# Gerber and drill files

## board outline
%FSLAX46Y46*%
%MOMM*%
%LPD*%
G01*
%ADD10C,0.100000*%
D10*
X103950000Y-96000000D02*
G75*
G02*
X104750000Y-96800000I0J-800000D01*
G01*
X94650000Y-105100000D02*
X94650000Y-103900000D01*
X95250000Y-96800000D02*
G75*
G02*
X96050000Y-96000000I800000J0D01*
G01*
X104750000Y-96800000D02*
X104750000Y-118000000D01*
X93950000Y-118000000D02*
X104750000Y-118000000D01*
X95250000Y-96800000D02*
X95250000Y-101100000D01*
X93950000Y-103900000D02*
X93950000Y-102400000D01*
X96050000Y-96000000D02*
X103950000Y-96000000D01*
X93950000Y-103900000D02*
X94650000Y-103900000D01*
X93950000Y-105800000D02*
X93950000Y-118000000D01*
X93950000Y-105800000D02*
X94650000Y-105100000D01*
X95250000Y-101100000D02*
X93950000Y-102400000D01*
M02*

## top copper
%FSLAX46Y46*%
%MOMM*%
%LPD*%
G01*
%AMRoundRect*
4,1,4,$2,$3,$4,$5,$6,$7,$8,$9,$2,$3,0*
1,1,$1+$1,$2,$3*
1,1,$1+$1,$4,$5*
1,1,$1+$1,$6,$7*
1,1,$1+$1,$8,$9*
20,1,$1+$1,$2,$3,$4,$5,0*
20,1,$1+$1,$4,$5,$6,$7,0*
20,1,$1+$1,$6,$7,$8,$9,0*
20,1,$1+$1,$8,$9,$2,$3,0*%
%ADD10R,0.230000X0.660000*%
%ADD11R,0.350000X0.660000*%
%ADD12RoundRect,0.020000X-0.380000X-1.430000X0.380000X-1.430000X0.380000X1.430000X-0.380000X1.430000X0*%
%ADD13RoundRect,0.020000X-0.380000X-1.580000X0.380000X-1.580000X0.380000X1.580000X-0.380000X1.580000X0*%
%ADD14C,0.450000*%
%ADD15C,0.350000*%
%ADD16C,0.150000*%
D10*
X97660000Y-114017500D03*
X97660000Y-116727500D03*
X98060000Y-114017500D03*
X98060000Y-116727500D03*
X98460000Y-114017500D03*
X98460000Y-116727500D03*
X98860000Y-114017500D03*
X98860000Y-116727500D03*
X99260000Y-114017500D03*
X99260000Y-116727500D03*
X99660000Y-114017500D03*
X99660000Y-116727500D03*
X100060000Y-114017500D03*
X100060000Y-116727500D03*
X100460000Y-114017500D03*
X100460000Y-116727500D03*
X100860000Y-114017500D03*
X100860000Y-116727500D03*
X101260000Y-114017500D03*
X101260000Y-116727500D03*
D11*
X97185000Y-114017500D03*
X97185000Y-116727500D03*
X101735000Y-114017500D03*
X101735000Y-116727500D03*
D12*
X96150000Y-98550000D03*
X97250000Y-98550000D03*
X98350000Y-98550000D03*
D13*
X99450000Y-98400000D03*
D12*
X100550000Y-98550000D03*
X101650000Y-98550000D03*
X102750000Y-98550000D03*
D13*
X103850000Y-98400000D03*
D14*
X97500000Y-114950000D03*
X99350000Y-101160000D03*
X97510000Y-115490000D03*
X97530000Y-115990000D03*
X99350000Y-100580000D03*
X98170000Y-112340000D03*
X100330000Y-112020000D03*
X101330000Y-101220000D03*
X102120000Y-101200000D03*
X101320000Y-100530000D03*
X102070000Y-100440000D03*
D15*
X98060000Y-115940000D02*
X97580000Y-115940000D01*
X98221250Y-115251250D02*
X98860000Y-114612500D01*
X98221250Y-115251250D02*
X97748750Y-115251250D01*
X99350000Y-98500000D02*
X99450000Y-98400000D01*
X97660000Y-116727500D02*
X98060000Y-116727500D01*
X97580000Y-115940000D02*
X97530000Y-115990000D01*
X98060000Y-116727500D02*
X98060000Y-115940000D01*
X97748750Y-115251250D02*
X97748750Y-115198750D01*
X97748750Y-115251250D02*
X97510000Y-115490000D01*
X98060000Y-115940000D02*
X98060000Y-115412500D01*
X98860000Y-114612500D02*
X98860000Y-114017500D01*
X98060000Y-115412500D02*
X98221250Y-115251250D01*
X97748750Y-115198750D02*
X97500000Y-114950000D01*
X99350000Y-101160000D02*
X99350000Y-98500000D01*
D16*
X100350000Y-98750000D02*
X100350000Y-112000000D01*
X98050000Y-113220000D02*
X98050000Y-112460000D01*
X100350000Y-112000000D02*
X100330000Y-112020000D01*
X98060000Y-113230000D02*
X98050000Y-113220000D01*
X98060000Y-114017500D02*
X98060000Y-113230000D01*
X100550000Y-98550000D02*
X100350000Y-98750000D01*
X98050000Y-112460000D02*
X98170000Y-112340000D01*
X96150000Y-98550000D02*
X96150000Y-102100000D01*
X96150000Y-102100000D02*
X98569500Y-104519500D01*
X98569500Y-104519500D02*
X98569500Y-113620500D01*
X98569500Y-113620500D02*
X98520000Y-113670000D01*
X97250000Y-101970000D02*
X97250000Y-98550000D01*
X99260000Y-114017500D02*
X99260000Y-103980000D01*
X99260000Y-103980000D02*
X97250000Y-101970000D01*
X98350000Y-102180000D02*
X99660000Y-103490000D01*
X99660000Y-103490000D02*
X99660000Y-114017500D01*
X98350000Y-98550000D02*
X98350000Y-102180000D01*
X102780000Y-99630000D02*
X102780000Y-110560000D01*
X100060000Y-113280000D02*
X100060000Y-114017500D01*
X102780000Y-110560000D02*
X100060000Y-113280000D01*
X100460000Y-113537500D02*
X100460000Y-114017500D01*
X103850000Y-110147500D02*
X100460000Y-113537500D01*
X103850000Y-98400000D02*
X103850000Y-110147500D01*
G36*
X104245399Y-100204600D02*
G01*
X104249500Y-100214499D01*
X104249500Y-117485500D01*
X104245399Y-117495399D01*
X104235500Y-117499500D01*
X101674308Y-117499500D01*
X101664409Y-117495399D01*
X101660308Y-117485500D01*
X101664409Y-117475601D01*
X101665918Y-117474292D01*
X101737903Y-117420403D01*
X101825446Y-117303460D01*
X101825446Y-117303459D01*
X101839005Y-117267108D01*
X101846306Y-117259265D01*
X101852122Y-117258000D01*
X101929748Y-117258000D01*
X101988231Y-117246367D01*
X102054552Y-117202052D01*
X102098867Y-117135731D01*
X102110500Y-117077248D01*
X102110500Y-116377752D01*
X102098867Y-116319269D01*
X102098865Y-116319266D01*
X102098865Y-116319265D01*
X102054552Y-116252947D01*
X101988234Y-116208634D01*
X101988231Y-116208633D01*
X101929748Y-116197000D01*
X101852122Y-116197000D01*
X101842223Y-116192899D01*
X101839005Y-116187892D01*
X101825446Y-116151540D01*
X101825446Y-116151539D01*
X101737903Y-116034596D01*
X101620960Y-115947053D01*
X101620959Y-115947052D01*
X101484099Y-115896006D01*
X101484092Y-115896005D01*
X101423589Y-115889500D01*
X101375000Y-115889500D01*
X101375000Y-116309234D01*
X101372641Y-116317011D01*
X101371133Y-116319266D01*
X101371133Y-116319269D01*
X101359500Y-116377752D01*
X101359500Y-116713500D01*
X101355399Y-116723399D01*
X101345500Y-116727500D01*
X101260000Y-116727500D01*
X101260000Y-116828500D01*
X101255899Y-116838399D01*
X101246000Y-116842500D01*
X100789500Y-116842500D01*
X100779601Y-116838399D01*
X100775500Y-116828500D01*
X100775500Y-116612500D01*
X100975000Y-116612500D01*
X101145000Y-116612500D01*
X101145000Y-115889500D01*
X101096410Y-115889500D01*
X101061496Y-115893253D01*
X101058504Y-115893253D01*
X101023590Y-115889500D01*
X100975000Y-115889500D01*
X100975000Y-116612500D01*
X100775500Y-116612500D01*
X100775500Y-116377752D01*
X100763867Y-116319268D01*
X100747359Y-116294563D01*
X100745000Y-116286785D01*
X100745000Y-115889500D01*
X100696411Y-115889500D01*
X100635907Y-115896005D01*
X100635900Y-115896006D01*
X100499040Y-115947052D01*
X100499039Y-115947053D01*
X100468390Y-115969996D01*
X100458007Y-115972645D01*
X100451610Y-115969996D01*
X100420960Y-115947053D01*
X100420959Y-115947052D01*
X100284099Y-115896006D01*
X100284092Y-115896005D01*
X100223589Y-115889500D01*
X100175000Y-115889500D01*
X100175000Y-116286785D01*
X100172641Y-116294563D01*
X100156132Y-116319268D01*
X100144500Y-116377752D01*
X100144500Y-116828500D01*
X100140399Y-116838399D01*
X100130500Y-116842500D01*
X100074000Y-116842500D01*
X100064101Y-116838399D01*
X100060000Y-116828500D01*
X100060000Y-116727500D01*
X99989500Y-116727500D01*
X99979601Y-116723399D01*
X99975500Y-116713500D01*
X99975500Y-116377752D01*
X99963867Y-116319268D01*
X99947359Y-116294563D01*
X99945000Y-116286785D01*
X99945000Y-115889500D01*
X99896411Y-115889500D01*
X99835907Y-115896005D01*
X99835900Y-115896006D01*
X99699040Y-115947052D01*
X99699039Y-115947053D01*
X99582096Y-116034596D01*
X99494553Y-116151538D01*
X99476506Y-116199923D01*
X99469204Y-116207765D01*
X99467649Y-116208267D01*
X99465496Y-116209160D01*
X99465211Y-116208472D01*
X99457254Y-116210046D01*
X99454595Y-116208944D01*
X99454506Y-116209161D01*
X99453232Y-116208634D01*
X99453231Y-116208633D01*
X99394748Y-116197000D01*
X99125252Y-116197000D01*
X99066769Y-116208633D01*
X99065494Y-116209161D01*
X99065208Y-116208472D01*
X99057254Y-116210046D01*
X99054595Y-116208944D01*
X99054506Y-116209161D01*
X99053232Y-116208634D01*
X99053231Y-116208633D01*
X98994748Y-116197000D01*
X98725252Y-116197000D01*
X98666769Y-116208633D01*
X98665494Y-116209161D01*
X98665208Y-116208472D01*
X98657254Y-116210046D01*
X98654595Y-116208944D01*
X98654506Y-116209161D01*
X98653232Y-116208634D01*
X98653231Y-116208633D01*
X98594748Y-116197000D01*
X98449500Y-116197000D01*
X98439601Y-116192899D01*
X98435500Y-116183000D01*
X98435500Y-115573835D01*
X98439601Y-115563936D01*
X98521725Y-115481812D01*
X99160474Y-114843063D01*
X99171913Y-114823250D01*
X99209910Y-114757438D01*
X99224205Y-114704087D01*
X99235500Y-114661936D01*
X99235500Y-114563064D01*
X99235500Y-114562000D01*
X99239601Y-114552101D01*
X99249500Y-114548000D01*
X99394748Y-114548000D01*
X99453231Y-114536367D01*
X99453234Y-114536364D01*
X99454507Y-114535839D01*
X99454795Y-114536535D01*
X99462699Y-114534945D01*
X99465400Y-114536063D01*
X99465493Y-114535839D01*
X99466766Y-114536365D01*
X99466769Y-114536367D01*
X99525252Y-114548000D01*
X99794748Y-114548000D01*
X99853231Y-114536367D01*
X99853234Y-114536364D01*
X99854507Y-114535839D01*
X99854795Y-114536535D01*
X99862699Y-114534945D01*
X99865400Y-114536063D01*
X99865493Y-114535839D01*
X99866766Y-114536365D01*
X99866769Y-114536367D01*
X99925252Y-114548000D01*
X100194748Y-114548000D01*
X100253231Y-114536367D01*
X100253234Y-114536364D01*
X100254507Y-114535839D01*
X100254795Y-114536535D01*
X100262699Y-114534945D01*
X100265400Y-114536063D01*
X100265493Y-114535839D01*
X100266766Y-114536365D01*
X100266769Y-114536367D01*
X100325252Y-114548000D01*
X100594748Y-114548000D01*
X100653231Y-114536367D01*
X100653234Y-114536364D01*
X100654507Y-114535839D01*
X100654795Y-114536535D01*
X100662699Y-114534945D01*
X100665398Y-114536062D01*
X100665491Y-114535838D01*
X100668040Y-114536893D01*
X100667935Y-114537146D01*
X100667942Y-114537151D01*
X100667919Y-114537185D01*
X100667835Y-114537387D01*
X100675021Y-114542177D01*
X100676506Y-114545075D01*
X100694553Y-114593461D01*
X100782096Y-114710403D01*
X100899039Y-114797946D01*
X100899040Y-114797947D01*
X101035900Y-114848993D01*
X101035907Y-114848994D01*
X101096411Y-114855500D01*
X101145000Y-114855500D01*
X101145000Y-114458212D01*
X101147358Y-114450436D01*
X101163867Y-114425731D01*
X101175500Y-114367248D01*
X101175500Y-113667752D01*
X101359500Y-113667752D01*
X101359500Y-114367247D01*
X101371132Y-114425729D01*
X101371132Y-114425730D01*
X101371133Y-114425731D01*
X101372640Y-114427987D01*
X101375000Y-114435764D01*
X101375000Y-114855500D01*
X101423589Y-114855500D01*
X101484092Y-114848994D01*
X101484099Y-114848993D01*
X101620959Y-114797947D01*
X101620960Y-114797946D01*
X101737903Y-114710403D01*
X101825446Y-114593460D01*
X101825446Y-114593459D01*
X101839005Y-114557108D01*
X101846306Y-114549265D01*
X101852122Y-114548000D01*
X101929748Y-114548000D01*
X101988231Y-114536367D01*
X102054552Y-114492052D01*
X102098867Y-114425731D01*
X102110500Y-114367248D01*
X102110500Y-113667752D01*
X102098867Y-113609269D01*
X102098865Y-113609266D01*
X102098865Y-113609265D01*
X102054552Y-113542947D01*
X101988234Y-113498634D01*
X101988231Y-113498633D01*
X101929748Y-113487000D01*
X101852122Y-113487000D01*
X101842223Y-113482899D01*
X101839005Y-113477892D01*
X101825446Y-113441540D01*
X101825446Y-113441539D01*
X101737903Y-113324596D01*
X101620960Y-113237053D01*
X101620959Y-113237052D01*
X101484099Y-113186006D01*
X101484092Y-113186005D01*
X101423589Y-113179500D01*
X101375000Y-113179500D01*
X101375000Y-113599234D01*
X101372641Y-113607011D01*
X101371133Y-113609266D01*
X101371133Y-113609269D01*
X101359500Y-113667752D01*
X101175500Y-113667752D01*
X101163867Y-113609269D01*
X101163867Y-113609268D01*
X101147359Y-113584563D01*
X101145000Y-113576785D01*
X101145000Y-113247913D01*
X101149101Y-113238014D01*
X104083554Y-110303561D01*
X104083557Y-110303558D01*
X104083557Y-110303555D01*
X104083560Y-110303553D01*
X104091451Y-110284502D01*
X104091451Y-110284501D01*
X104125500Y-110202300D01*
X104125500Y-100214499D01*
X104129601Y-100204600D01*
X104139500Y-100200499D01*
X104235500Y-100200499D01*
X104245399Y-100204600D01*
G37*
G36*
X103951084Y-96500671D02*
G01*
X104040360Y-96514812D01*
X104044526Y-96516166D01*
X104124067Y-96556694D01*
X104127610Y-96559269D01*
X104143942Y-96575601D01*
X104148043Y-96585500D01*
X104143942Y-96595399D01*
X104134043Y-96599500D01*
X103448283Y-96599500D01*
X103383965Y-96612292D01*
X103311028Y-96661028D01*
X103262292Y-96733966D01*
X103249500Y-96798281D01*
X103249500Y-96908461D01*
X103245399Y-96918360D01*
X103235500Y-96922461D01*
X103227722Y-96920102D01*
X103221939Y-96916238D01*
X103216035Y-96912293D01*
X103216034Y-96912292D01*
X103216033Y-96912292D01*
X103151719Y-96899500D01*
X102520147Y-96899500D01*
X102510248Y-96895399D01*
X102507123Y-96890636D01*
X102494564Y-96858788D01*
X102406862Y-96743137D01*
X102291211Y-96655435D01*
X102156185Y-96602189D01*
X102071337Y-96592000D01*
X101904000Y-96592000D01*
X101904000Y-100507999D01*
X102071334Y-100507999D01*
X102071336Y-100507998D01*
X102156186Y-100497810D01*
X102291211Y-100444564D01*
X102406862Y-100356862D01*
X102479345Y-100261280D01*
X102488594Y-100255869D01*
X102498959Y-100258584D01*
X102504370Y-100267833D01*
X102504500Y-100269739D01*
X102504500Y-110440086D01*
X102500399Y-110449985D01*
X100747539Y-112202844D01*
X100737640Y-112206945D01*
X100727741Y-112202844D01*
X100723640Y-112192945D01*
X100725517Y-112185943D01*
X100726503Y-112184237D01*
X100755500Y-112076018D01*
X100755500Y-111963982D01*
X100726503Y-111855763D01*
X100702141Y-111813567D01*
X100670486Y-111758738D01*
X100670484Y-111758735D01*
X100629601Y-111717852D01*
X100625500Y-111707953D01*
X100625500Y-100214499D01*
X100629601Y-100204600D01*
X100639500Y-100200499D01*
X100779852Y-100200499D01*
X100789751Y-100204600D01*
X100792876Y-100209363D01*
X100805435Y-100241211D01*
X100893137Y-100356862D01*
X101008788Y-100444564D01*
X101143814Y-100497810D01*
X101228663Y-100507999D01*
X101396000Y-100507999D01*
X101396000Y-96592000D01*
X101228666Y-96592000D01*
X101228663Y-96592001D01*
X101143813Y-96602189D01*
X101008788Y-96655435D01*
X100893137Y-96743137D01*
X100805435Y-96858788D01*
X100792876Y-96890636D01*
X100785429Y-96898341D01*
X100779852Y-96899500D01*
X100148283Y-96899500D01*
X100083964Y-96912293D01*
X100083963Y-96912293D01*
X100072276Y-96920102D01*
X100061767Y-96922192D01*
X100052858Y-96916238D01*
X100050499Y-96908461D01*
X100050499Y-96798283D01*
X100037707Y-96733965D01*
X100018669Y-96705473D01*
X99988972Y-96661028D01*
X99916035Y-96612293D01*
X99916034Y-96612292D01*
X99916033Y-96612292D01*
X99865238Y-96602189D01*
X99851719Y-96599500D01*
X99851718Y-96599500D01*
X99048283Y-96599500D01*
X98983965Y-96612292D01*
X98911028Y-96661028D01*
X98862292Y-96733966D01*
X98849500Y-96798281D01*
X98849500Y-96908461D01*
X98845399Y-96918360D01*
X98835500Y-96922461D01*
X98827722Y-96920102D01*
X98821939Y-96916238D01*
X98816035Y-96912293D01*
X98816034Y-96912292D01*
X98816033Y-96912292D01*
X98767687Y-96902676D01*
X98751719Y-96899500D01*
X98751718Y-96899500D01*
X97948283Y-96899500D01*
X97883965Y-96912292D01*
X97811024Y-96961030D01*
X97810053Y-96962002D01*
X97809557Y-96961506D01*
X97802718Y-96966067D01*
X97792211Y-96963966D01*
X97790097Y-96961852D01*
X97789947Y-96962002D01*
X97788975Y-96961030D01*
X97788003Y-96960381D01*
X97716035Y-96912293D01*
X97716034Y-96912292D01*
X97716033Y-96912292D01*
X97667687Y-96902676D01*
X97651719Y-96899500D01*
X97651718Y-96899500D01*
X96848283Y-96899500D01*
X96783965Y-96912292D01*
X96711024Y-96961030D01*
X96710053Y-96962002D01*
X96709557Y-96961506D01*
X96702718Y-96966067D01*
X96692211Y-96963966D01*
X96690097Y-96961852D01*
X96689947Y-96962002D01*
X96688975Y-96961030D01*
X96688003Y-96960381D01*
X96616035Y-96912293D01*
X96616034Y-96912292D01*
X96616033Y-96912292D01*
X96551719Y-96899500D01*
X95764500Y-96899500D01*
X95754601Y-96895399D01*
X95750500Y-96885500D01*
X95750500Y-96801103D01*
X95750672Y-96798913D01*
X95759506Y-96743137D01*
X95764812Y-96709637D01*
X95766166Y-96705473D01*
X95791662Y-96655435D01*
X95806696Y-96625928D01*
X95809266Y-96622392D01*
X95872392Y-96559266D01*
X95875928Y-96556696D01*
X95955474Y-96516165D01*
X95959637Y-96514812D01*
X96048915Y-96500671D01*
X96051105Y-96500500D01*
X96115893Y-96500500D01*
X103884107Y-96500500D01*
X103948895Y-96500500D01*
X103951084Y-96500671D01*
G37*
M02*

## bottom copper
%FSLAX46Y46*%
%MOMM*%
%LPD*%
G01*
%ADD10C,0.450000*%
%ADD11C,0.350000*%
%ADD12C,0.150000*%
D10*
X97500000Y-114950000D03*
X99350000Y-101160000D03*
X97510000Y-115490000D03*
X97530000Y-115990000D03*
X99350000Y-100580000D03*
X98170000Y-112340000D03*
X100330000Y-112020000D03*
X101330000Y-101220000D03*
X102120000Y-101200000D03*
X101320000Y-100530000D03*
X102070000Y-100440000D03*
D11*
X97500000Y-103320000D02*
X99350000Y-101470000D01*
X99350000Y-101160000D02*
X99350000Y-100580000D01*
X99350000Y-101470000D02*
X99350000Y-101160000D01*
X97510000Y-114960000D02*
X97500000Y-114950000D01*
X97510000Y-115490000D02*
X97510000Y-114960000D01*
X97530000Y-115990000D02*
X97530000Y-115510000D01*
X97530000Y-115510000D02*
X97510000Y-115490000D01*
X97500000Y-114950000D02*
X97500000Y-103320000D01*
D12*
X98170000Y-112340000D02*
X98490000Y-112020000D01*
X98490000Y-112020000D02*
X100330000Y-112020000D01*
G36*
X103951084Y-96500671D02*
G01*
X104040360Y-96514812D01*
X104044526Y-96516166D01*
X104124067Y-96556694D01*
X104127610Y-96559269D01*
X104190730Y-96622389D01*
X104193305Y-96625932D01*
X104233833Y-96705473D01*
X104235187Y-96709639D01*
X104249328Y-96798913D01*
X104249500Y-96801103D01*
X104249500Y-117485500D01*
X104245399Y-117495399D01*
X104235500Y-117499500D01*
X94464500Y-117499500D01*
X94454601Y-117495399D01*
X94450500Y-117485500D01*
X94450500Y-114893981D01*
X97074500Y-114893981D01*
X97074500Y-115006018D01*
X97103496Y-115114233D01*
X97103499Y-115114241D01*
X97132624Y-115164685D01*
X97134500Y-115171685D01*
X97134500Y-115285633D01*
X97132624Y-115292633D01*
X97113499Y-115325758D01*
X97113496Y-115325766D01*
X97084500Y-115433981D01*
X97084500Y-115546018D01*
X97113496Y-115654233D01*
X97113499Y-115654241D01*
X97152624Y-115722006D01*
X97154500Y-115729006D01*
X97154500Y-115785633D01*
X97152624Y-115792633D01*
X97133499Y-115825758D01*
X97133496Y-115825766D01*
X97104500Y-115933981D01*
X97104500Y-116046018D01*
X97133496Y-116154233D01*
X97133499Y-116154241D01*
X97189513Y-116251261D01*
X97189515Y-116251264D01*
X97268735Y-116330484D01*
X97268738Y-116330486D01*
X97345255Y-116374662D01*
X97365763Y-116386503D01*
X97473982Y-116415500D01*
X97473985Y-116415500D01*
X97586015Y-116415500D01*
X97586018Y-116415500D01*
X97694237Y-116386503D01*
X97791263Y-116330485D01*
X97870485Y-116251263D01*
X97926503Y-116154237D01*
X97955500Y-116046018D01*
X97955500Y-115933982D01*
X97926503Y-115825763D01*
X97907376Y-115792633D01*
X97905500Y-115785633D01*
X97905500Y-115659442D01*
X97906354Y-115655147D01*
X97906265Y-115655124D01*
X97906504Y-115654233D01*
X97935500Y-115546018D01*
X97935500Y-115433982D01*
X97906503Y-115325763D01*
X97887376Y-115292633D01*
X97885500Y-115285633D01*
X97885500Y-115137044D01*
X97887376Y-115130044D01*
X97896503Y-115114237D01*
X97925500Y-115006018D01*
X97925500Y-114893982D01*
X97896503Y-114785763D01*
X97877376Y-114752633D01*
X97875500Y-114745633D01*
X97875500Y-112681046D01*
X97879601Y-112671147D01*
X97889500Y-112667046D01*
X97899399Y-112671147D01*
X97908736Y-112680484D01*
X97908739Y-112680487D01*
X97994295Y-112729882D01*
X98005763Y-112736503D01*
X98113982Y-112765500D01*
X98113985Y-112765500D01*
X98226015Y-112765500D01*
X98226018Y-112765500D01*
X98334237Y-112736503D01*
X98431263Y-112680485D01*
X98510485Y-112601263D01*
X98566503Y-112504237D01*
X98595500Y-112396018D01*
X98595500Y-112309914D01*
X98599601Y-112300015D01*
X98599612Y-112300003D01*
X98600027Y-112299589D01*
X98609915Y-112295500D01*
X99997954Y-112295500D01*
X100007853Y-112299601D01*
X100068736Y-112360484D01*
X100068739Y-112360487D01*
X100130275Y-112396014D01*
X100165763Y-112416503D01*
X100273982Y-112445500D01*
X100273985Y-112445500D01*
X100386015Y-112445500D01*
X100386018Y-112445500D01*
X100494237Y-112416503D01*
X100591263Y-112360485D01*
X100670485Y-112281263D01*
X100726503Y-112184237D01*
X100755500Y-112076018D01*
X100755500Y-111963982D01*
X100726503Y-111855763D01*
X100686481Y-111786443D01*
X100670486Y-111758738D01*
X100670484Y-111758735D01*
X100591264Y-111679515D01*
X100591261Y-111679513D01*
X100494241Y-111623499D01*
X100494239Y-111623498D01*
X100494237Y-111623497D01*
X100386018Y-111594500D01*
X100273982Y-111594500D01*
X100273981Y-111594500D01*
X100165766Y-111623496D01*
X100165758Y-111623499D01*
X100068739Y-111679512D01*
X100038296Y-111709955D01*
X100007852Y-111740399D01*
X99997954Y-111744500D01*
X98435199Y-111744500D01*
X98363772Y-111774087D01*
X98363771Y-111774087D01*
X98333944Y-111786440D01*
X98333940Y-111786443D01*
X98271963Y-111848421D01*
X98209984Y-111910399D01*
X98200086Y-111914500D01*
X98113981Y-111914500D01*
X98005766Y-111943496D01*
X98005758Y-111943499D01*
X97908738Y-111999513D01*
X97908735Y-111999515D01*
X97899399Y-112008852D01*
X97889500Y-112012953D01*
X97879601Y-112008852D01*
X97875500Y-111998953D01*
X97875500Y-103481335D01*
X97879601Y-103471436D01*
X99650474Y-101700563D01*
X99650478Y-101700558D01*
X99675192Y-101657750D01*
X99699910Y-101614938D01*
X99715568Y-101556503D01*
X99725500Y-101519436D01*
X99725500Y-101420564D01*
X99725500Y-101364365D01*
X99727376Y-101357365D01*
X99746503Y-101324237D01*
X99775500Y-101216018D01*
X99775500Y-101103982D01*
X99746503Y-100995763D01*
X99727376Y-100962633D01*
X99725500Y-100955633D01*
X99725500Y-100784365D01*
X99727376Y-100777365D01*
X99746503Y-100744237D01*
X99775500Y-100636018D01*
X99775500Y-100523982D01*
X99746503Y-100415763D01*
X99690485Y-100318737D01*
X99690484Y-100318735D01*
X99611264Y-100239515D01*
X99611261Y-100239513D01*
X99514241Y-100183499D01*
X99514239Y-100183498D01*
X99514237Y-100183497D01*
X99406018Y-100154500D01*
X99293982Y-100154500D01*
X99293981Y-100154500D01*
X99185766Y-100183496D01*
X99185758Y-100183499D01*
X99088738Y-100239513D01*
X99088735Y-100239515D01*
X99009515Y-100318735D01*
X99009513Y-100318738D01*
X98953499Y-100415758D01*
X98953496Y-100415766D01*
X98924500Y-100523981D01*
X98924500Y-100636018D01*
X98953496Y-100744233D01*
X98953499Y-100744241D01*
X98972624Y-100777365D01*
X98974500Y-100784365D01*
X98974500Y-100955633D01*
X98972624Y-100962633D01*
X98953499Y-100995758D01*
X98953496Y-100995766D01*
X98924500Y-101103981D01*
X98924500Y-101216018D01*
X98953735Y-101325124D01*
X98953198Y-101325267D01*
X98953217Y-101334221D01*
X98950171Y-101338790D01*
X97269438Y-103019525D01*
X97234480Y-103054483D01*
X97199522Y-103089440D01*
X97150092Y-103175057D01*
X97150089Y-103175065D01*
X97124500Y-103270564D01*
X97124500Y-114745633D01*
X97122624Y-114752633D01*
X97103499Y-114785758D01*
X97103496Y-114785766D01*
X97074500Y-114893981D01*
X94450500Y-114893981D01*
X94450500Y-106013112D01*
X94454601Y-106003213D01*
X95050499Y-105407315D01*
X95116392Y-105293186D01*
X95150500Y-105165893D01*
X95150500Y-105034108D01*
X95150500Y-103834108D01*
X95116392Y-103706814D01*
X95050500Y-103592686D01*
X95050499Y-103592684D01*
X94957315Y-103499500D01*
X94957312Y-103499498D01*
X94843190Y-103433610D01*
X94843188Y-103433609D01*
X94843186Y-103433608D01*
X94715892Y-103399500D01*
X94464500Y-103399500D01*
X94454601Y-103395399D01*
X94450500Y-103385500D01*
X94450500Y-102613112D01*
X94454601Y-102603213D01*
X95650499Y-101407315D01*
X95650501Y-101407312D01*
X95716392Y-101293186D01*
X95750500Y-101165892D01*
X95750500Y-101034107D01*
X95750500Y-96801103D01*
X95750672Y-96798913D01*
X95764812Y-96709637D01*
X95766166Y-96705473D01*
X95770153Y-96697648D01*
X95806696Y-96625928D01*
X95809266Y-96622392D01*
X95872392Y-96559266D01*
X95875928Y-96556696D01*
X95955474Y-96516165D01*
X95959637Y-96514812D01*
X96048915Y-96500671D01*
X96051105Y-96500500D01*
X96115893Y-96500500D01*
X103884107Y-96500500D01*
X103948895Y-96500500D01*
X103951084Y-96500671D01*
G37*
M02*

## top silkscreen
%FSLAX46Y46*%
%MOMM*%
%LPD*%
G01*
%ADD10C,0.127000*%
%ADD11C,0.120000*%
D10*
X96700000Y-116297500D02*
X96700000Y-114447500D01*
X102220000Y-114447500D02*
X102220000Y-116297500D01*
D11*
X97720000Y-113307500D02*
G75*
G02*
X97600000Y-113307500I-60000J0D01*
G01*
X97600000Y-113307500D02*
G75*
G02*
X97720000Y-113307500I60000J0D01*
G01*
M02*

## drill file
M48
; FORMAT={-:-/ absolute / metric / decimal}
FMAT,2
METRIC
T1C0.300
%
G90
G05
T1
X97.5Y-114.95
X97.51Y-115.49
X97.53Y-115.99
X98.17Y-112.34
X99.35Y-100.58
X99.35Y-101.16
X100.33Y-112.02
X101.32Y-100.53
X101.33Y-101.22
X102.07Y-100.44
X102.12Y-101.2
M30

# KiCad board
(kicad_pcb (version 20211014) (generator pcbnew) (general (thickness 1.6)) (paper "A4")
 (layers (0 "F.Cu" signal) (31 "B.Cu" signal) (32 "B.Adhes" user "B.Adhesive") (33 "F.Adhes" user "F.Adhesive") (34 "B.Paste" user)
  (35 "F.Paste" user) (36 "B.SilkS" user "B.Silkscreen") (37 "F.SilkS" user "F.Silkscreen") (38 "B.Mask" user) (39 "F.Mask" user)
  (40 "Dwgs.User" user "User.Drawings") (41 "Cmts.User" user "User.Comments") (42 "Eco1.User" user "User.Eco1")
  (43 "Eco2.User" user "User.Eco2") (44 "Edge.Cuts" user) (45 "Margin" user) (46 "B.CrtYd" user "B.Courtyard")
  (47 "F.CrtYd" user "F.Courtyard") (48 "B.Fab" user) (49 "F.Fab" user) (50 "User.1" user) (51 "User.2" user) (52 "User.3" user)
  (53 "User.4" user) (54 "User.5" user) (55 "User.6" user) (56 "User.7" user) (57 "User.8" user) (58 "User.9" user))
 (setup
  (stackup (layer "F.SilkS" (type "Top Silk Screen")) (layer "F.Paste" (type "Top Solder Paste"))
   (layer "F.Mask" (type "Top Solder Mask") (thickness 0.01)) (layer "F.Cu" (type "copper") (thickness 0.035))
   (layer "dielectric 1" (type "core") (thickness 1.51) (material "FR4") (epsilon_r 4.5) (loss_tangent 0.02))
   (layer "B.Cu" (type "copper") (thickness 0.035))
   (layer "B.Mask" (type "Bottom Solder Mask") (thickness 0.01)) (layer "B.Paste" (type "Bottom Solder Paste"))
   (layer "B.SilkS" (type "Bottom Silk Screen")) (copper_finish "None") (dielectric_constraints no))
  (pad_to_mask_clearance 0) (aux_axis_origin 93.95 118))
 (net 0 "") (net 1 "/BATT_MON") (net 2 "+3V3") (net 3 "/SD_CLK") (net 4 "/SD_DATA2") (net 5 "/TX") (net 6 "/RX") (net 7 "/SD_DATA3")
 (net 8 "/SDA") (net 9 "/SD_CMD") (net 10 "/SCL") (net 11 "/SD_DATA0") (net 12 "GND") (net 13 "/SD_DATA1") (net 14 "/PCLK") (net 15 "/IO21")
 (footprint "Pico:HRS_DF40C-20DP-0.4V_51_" (layer "F.Cu") (at 99.46 115.3725)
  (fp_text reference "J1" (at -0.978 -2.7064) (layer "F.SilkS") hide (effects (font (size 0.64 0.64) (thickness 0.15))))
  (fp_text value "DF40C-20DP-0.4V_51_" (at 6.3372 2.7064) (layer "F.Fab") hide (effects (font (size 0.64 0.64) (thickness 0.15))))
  (fp_line (start -2.76 0.925) (end -2.76 -0.925) (layer "F.SilkS") (width 0.127))
  (fp_line (start 2.76 -0.925) (end 2.76 0.925) (layer "F.SilkS") (width 0.127))
  (fp_circle (center -1.8 -2.065) (end -1.74 -2.065) (layer "F.SilkS") (width 0.12) (fill none))
  (pad "1" smd rect (at -1.8 -1.355) (size 0.23 0.66) (layers "F.Cu" "F.Paste" "F.Mask") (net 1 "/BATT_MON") (solder_mask_margin 0.102))
  (pad "2" smd rect (at -1.8 1.355) (size 0.23 0.66) (layers "F.Cu" "F.Paste" "F.Mask") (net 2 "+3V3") (solder_mask_margin 0.102))
  (pad "3" smd rect (at -1.4 -1.355) (size 0.23 0.66) (layers "F.Cu" "F.Paste" "F.Mask") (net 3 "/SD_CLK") (solder_mask_margin 0.102))
  (pad "4" smd rect (at -1.4 1.355) (size 0.23 0.66) (layers "F.Cu" "F.Paste" "F.Mask") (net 2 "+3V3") (solder_mask_margin 0.102))
  (pad "5" smd rect (at -1 -1.355) (size 0.23 0.66) (layers "F.Cu" "F.Paste" "F.Mask") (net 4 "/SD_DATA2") (solder_mask_margin 0.102))
  (pad "6" smd rect (at -1 1.355) (size 0.23 0.66) (layers "F.Cu" "F.Paste" "F.Mask") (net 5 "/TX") (solder_mask_margin 0.102))
  (pad "7" smd rect (at -0.6 -1.355) (size 0.23 0.66) (layers "F.Cu" "F.Paste" "F.Mask") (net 2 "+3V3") (solder_mask_margin 0.102))
  (pad "8" smd rect (at -0.6 1.355) (size 0.23 0.66) (layers "F.Cu" "F.Paste" "F.Mask") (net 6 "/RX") (solder_mask_margin 0.102))
  (pad "9" smd rect (at -0.2 -1.355) (size 0.23 0.66) (layers "F.Cu" "F.Paste" "F.Mask") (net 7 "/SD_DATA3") (solder_mask_margin 0.102))
  (pad "10" smd rect (at -0.2 1.355) (size 0.23 0.66) (layers "F.Cu" "F.Paste" "F.Mask") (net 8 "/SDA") (solder_mask_margin 0.102))
  (pad "11" smd rect (at 0.2 -1.355) (size 0.23 0.66) (layers "F.Cu" "F.Paste" "F.Mask") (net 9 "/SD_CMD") (solder_mask_margin 0.102))
  (pad "12" smd rect (at 0.2 1.355) (size 0.23 0.66) (layers "F.Cu" "F.Paste" "F.Mask") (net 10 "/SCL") (solder_mask_margin 0.102))
  (pad "13" smd rect (at 0.6 -1.355) (size 0.23 0.66) (layers "F.Cu" "F.Paste" "F.Mask") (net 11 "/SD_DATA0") (solder_mask_margin 0.102))
  (pad "14" smd rect (at 0.6 1.355) (size 0.23 0.66) (layers "F.Cu" "F.Paste" "F.Mask") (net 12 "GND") (solder_mask_margin 0.102))
  (pad "15" smd rect (at 1 -1.355) (size 0.23 0.66) (layers "F.Cu" "F.Paste" "F.Mask") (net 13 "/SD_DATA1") (solder_mask_margin 0.102))
  (pad "16" smd rect (at 1 1.355) (size 0.23 0.66) (layers "F.Cu" "F.Paste" "F.Mask") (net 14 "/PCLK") (solder_mask_margin 0.102))
  (pad "17" smd rect (at 1.4 -1.355) (size 0.23 0.66) (layers "F.Cu" "F.Paste" "F.Mask") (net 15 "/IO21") (solder_mask_margin 0.102))
  (pad "18" smd rect (at 1.4 1.355) (size 0.23 0.66) (layers "F.Cu" "F.Paste" "F.Mask") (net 12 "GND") (solder_mask_margin 0.102))
  (pad "19" smd rect (at 1.8 -1.355) (size 0.23 0.66) (layers "F.Cu" "F.Paste" "F.Mask") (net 12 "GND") (solder_mask_margin 0.102))
  (pad "20" smd rect (at 1.8 1.355) (size 0.23 0.66) (layers "F.Cu" "F.Paste" "F.Mask") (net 12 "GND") (solder_mask_margin 0.102))
  (pad "S1" smd rect (at -2.275 -1.355) (size 0.35 0.66) (layers "F.Cu" "F.Paste" "F.Mask") (solder_mask_margin 0.102))
  (pad "S2" smd rect (at -2.275 1.355) (size 0.35 0.66) (layers "F.Cu" "F.Paste" "F.Mask") (solder_mask_margin 0.102))
  (pad "S3" smd rect (at 2.275 -1.355) (size 0.35 0.66) (layers "F.Cu" "F.Paste" "F.Mask") (solder_mask_margin 0.102))
  (pad "S4" smd rect (at 2.275 1.355) (size 0.35 0.66) (layers "F.Cu" "F.Paste" "F.Mask") (solder_mask_margin 0.102)))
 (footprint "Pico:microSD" (layer "F.Cu") (at 100 100)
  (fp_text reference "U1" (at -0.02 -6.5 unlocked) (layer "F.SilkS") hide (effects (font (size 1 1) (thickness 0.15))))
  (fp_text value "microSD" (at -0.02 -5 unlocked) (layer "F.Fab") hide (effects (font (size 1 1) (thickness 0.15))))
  (pad "1" smd roundrect (at -3.85 -1.45) (size 0.8 2.9) (layers "F.Cu" "F.Paste" "F.Mask") (roundrect_rratio 0.025) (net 4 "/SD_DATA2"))
  (pad "2" smd roundrect (at -2.75 -1.45) (size 0.8 2.9) (layers "F.Cu" "F.Paste" "F.Mask") (roundrect_rratio 0.025) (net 7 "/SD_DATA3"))
  (pad "3" smd roundrect (at -1.65 -1.45) (size 0.8 2.9) (layers "F.Cu" "F.Paste" "F.Mask") (roundrect_rratio 0.025) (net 9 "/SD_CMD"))
  (pad "4" smd roundrect (at -0.55 -1.6) (size 0.8 3.2) (layers "F.Cu" "F.Paste" "F.Mask") (roundrect_rratio 0.025) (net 2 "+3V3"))
  (pad "5" smd roundrect (at 0.55 -1.45) (size 0.8 2.9) (layers "F.Cu" "F.Paste" "F.Mask") (roundrect_rratio 0.025) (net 3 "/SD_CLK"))
  (pad "6" smd roundrect (at 1.65 -1.45) (size 0.8 2.9) (layers "F.Cu" "F.Paste" "F.Mask") (roundrect_rratio 0.025) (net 12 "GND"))
  (pad "7" smd roundrect (at 2.75 -1.45) (size 0.8 2.9) (layers "F.Cu" "F.Paste" "F.Mask") (roundrect_rratio 0.025) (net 11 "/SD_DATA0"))
  (pad "8" smd roundrect (at 3.85 -1.6) (size 0.8 3.2) (layers "F.Cu" "F.Paste" "F.Mask") (roundrect_rratio 0.025) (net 13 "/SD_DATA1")))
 (gr_arc (start 103.95 96) (mid 104.515685 96.234315) (end 104.75 96.8) (layer "Edge.Cuts") (width 0.1))
 (gr_line (start 94.65 105.1) (end 94.65 103.9) (layer "Edge.Cuts") (width 0.1))
 (gr_arc (start 95.25 96.8) (mid 95.484315 96.234315) (end 96.05 96) (layer "Edge.Cuts") (width 0.1))
 (gr_line (start 104.75 96.8) (end 104.75 118) (layer "Edge.Cuts") (width 0.1))
 (gr_line (start 93.95 118) (end 104.75 118) (layer "Edge.Cuts") (width 0.1))
 (gr_line locked (start 95.25 96.8) (end 95.25 101.1) (layer "Edge.Cuts") (width 0.1))
 (gr_line (start 93.95 103.9) (end 93.95 102.4) (layer "Edge.Cuts") (width 0.1))
 (gr_line (start 96.05 96) (end 103.95 96) (layer "Edge.Cuts") (width 0.1))
 (gr_line (start 93.95 103.9) (end 94.65 103.9) (layer "Edge.Cuts") (width 0.1))
 (gr_line (start 93.95 105.8) (end 93.95 118) (layer "Edge.Cuts") (width 0.1))
 (gr_line (start 93.95 105.8) (end 94.65 105.1) (layer "Edge.Cuts") (width 0.1))
 (gr_line (start 95.25 101.1) (end 93.95 102.4) (layer "Edge.Cuts") (width 0.1))
 (segment (start 98.06 115.94) (end 97.58 115.94) (width 0.35) (layer "F.Cu") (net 2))
 (segment (start 98.22125 115.25125) (end 98.86 114.6125) (width 0.35) (layer "F.Cu") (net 2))
 (segment (start 98.22125 115.25125) (end 97.74875 115.25125) (width 0.35) (layer "F.Cu") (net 2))
 (segment (start 99.35 98.5) (end 99.45 98.4) (width 0.35) (layer "F.Cu") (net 2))
 (segment (start 97.66 116.7275) (end 98.06 116.7275) (width 0.35) (layer "F.Cu") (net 2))
 (segment (start 97.58 115.94) (end 97.53 115.99) (width 0.35) (layer "F.Cu") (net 2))
 (segment (start 98.06 116.7275) (end 98.06 115.94) (width 0.35) (layer "F.Cu") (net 2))
 (segment (start 97.74875 115.25125) (end 97.74875 115.19875) (width 0.35) (layer "F.Cu") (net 2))
 (segment (start 97.74875 115.25125) (end 97.51 115.49) (width 0.35) (layer "F.Cu") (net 2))
 (segment (start 98.06 115.94) (end 98.06 115.4125) (width 0.35) (layer "F.Cu") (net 2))
 (segment (start 98.86 114.6125) (end 98.86 114.0175) (width 0.35) (layer "F.Cu") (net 2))
 (segment (start 98.06 115.4125) (end 98.22125 115.25125) (width 0.35) (layer "F.Cu") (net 2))
 (segment (start 97.74875 115.19875) (end 97.5 114.95) (width 0.35) (layer "F.Cu") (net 2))
 (segment (start 99.35 101.16) (end 99.35 98.5) (width 0.35) (layer "F.Cu") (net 2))
 (via (at 97.5 114.95) (size 0.45) (drill 0.3) (layers "F.Cu" "B.Cu") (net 2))
 (via (at 99.35 101.16) (size 0.45) (drill 0.3) (layers "F.Cu" "B.Cu") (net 2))
 (via (at 97.51 115.49) (size 0.45) (drill 0.3) (layers "F.Cu" "B.Cu") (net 2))
 (via (at 97.53 115.99) (size 0.45) (drill 0.3) (layers "F.Cu" "B.Cu") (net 2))
 (via (at 99.35 100.58) (size 0.45) (drill 0.3) (layers "F.Cu" "B.Cu") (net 2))
 (segment (start 97.5 103.32) (end 99.35 101.47) (width 0.35) (layer "B.Cu") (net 2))
 (segment (start 99.35 101.16) (end 99.35 100.58) (width 0.35) (layer "B.Cu") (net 2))
 (segment (start 99.35 101.47) (end 99.35 101.16) (width 0.35) (layer "B.Cu") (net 2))
 (segment (start 97.51 114.96) (end 97.5 114.95) (width 0.35) (layer "B.Cu") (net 2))
 (segment (start 97.51 115.49) (end 97.51 114.96) (width 0.35) (layer "B.Cu") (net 2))
 (segment (start 97.53 115.99) (end 97.53 115.51) (width 0.35) (layer "B.Cu") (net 2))
 (segment (start 97.53 115.51) (end 97.51 115.49) (width 0.35) (layer "B.Cu") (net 2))
 (segment (start 97.5 114.95) (end 97.5 103.32) (width 0.35) (layer "B.Cu") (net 2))
 (segment (start 100.35 98.75) (end 100.35 112) (width 0.15) (layer "F.Cu") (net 3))
 (segment (start 98.05 113.22) (end 98.05 112.46) (width 0.15) (layer "F.Cu") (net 3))
 (segment (start 100.35 112) (end 100.33 112.02) (width 0.15) (layer "F.Cu") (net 3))
 (segment (start 98.06 113.23) (end 98.05 113.22) (width 0.15) (layer "F.Cu") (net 3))
 (segment (start 98.06 114.0175) (end 98.06 113.23) (width 0.15) (layer "F.Cu") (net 3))
 (segment (start 100.55 98.55) (end 100.35 98.75) (width 0.15) (layer "F.Cu") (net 3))
 (segment (start 98.05 112.46) (end 98.17 112.34) (width 0.15) (layer "F.Cu") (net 3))
 (via (at 98.17 112.34) (size 0.45) (drill 0.3) (layers "F.Cu" "B.Cu") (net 3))
 (via (at 100.33 112.02) (size 0.45) (drill 0.3) (layers "F.Cu" "B.Cu") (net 3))
 (segment (start 98.17 112.34) (end 98.49 112.02) (width 0.15) (layer "B.Cu") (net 3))
 (segment (start 98.49 112.02) (end 100.33 112.02) (width 0.15) (layer "B.Cu") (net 3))
 (segment (start 96.15 98.55) (end 96.15 102.1) (width 0.15) (layer "F.Cu") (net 4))
 (segment (start 96.15 102.1) (end 98.5695 104.5195) (width 0.15) (layer "F.Cu") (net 4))
 (segment (start 98.5695 104.5195) (end 98.5695 113.6205) (width 0.15) (layer "F.Cu") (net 4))
 (segment (start 98.5695 113.6205) (end 98.52 113.67) (width 0.15) (layer "F.Cu") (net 4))
 (segment (start 97.25 101.97) (end 97.25 98.55) (width 0.15) (layer "F.Cu") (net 7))
 (segment (start 99.26 114.0175) (end 99.26 103.98) (width 0.15) (layer "F.Cu") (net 7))
 (segment (start 99.26 103.98) (end 97.25 101.97) (width 0.15) (layer "F.Cu") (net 7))
 (segment (start 98.35 102.18) (end 99.66 103.49) (width 0.15) (layer "F.Cu") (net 9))
 (segment (start 99.66 103.49) (end 99.66 114.0175) (width 0.15) (layer "F.Cu") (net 9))
 (segment (start 98.35 98.55) (end 98.35 102.18) (width 0.15) (layer "F.Cu") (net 9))
 (segment (start 102.78 99.63) (end 102.78 110.56) (width 0.15) (layer "F.Cu") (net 11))
 (segment (start 100.06 113.28) (end 100.06 114.0175) (width 0.15) (layer "F.Cu") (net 11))
 (segment (start 102.78 110.56) (end 100.06 113.28) (width 0.15) (layer "F.Cu") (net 11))
 (via (at 101.33 101.22) (size 0.45) (drill 0.3) (layers "F.Cu" "B.Cu") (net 12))
 (via (at 102.12 101.2) (size 0.45) (drill 0.3) (layers "F.Cu" "B.Cu") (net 12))
 (via (at 101.32 100.53) (size 0.45) (drill 0.3) (layers "F.Cu" "B.Cu") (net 12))
 (via (at 102.07 100.44) (size 0.45) (drill 0.3) (layers "F.Cu" "B.Cu") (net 12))
 (segment (start 100.46 113.5375) (end 100.46 114.0175) (width 0.15) (layer "F.Cu") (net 13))
 (segment (start 103.85 110.1475) (end 100.46 113.5375) (width 0.15) (layer "F.Cu") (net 13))
 (segment (start 103.85 98.4) (end 103.85 110.1475) (width 0.15) (layer "F.Cu") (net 13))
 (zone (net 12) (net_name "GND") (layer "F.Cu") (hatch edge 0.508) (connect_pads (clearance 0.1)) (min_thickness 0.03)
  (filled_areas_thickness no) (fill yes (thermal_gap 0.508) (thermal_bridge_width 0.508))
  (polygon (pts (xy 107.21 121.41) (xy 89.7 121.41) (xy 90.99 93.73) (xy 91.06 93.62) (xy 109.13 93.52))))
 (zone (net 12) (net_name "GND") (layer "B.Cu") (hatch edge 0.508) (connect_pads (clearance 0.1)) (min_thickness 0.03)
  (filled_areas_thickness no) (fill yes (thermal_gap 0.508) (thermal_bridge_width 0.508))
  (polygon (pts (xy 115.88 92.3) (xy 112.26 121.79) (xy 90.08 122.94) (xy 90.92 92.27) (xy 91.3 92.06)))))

